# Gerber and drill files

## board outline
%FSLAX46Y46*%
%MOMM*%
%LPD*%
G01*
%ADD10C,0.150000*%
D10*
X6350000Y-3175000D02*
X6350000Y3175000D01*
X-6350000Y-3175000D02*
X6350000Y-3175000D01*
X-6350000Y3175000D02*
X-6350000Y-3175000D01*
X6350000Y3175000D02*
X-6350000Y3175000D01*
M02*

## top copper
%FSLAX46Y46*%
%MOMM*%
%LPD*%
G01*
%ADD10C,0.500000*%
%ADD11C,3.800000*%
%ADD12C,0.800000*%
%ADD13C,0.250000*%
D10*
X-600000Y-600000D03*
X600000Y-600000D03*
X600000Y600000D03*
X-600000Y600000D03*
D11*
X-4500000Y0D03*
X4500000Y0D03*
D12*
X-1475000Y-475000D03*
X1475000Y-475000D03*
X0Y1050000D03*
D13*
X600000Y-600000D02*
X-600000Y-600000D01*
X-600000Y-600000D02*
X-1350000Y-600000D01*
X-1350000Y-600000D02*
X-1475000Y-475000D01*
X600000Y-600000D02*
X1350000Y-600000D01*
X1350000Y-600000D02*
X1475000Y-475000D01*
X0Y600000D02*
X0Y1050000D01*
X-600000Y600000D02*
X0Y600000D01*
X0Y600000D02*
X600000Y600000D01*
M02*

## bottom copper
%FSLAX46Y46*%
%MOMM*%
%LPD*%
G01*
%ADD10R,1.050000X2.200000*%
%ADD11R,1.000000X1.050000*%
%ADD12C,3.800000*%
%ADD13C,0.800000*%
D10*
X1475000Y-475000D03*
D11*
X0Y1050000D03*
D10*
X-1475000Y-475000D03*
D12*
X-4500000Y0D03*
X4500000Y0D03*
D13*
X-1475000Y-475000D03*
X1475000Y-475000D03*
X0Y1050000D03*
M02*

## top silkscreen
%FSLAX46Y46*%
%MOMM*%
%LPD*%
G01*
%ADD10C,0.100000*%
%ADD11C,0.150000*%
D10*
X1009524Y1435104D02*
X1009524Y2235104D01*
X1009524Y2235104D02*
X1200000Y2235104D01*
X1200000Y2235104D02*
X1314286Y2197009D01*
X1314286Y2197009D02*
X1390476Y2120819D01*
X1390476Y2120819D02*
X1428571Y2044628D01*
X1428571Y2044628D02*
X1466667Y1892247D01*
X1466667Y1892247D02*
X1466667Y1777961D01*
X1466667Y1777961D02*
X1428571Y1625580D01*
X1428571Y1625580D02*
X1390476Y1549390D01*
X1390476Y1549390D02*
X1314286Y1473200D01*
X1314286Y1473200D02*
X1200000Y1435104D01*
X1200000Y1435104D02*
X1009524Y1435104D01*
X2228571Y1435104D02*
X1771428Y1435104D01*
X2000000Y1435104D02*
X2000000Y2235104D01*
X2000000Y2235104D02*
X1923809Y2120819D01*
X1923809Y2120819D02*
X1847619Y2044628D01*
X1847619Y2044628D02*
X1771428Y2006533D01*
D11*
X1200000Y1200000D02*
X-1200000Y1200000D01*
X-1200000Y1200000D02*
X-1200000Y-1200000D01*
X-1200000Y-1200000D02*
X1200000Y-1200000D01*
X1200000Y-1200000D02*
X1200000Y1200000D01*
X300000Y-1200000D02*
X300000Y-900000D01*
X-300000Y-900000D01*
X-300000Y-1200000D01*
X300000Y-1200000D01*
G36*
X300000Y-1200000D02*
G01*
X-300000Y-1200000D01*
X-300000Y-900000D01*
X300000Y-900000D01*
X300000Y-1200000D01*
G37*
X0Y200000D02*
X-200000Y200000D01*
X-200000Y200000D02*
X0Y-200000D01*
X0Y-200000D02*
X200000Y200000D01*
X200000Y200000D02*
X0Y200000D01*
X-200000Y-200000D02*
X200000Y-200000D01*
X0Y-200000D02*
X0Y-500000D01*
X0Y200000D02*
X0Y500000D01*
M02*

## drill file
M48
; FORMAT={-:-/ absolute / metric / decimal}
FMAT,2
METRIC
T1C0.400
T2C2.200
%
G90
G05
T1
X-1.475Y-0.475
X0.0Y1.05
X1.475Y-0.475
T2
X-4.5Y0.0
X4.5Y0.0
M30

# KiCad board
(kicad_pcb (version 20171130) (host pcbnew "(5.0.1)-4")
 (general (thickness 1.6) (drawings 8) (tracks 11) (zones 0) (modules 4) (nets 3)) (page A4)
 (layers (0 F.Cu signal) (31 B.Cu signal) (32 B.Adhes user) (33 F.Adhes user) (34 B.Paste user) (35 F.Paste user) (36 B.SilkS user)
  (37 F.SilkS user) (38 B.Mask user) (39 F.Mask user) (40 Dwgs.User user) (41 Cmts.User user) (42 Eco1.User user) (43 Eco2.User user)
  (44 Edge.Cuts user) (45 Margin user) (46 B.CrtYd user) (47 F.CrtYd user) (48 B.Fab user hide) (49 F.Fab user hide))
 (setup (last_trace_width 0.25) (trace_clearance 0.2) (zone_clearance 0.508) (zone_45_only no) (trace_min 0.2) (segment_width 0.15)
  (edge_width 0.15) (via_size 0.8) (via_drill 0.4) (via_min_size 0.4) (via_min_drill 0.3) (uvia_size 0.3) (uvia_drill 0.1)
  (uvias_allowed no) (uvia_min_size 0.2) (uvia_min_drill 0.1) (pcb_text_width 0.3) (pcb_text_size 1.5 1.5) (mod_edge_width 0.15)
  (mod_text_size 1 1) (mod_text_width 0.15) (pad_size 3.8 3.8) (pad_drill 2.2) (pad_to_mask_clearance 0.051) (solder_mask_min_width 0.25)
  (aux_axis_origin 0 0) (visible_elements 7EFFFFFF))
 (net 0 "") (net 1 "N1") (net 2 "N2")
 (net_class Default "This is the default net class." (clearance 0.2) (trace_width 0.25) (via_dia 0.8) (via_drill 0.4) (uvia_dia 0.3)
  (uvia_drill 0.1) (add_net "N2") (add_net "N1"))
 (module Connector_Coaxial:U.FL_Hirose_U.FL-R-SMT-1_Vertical (layer B.Cu) (at 0 0 270)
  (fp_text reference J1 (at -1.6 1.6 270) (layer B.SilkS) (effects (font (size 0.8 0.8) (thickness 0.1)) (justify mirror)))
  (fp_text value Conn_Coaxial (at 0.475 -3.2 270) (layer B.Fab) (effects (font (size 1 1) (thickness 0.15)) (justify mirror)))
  (pad 2 smd rect (at 0.475 -1.475 270) (size 2.2 1.05) (layers B.Cu B.Paste B.Mask) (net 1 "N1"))
  (pad 1 smd rect (at -1.05 0 270) (size 1.05 1) (layers B.Cu B.Paste B.Mask) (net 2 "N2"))
  (pad 2 smd rect (at 0.475 1.475 270) (size 2.2 1.05) (layers B.Cu B.Paste B.Mask) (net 1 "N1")))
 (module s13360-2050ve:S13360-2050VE (layer F.Cu) (at 0 0)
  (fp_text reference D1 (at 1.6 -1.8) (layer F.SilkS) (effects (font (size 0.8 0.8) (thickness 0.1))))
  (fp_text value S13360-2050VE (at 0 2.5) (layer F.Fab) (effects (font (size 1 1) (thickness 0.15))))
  (fp_line (start 1.2 -1.2) (end -1.2 -1.2) (layer F.SilkS) (width 0.15))
  (fp_line (start -1.2 -1.2) (end -1.2 1.2) (layer F.SilkS) (width 0.15))
  (fp_line (start -1.2 1.2) (end 1.2 1.2) (layer F.SilkS) (width 0.15))
  (fp_line (start 1.2 1.2) (end 1.2 -1.2) (layer F.SilkS) (width 0.15))
  (fp_poly (pts (xy 0.3 1.2) (xy 0.3 0.9) (xy -0.3 0.9) (xy -0.3 1.2)) (layer F.SilkS) (width 0.15))
  (fp_line (start 0 -0.2) (end -0.2 -0.2) (layer F.SilkS) (width 0.15))
  (fp_line (start -0.2 -0.2) (end 0 0.2) (layer F.SilkS) (width 0.15))
  (fp_line (start 0 0.2) (end 0.2 -0.2) (layer F.SilkS) (width 0.15))
  (fp_line (start 0.2 -0.2) (end 0 -0.2) (layer F.SilkS) (width 0.15))
  (fp_line (start -0.2 0.2) (end 0.2 0.2) (layer F.SilkS) (width 0.15))
  (fp_line (start 0 0.2) (end 0 0.5) (layer F.SilkS) (width 0.15))
  (fp_line (start 0 -0.2) (end 0 -0.5) (layer F.SilkS) (width 0.15))
  (pad 2 smd circle (at -0.6 0.6) (size 0.5 0.5) (layers F.Cu F.Paste F.Mask) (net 1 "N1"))
  (pad 2 smd circle (at 0.6 0.6) (size 0.5 0.5) (layers F.Cu F.Paste F.Mask) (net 1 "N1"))
  (pad 1 smd circle (at 0.6 -0.6) (size 0.5 0.5) (layers F.Cu F.Paste F.Mask) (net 2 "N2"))
  (pad 1 smd circle (at -0.6 -0.6) (size 0.5 0.5) (layers F.Cu F.Paste F.Mask) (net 2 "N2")))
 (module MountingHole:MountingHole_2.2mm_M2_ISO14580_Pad (layer F.Cu) (at -4.5 0)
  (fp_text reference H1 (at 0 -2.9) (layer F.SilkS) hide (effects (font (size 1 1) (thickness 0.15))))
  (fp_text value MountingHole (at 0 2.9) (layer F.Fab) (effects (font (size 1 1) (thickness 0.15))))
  (pad 1 thru_hole circle (at 0 0) (size 3.8 3.8) (drill 2.2) (layers *.Cu *.Mask)))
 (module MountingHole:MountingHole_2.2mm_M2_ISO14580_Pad (layer F.Cu) (at 4.5 0)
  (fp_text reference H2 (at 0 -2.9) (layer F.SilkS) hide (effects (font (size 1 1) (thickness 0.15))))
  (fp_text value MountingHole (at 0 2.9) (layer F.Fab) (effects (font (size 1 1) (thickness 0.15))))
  (pad 1 thru_hole circle (at 0 0) (size 3.8 3.8) (drill 2.2) (layers *.Cu *.Mask)))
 (gr_line (start 6.35 3.175) (end 6.35 -3.175) (layer Edge.Cuts) (width 0.15))
 (gr_line (start -6.35 3.175) (end 6.35 3.175) (layer Edge.Cuts) (width 0.15))
 (gr_line (start -6.35 -3.175) (end -6.35 3.175) (layer Edge.Cuts) (width 0.15))
 (gr_line (start 6.35 -3.175) (end -6.35 -3.175) (layer Edge.Cuts) (width 0.15))
 (segment (start 0.6 0.6) (end -0.6 0.6) (width 0.25) (layer F.Cu) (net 1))
 (via (at -1.475 0.475) (size 0.8) (drill 0.4) (layers F.Cu B.Cu) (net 1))
 (segment (start -0.6 0.6) (end -1.35 0.6) (width 0.25) (layer F.Cu) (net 1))
 (segment (start -1.35 0.6) (end -1.475 0.475) (width 0.25) (layer F.Cu) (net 1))
 (via (at 1.475 0.475) (size 0.8) (drill 0.4) (layers F.Cu B.Cu) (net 1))
 (segment (start 0.6 0.6) (end 1.35 0.6) (width 0.25) (layer F.Cu) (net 1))
 (segment (start 1.35 0.6) (end 1.475 0.475) (width 0.25) (layer F.Cu) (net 1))
 (via (at 0 -1.05) (size 0.8) (drill 0.4) (layers F.Cu B.Cu) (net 2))
 (segment (start 0 -0.6) (end 0 -1.05) (width 0.25) (layer F.Cu) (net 2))
 (segment (start -0.6 -0.6) (end 0 -0.6) (width 0.25) (layer F.Cu) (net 2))
 (segment (start 0 -0.6) (end 0.6 -0.6) (width 0.25) (layer F.Cu) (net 2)))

